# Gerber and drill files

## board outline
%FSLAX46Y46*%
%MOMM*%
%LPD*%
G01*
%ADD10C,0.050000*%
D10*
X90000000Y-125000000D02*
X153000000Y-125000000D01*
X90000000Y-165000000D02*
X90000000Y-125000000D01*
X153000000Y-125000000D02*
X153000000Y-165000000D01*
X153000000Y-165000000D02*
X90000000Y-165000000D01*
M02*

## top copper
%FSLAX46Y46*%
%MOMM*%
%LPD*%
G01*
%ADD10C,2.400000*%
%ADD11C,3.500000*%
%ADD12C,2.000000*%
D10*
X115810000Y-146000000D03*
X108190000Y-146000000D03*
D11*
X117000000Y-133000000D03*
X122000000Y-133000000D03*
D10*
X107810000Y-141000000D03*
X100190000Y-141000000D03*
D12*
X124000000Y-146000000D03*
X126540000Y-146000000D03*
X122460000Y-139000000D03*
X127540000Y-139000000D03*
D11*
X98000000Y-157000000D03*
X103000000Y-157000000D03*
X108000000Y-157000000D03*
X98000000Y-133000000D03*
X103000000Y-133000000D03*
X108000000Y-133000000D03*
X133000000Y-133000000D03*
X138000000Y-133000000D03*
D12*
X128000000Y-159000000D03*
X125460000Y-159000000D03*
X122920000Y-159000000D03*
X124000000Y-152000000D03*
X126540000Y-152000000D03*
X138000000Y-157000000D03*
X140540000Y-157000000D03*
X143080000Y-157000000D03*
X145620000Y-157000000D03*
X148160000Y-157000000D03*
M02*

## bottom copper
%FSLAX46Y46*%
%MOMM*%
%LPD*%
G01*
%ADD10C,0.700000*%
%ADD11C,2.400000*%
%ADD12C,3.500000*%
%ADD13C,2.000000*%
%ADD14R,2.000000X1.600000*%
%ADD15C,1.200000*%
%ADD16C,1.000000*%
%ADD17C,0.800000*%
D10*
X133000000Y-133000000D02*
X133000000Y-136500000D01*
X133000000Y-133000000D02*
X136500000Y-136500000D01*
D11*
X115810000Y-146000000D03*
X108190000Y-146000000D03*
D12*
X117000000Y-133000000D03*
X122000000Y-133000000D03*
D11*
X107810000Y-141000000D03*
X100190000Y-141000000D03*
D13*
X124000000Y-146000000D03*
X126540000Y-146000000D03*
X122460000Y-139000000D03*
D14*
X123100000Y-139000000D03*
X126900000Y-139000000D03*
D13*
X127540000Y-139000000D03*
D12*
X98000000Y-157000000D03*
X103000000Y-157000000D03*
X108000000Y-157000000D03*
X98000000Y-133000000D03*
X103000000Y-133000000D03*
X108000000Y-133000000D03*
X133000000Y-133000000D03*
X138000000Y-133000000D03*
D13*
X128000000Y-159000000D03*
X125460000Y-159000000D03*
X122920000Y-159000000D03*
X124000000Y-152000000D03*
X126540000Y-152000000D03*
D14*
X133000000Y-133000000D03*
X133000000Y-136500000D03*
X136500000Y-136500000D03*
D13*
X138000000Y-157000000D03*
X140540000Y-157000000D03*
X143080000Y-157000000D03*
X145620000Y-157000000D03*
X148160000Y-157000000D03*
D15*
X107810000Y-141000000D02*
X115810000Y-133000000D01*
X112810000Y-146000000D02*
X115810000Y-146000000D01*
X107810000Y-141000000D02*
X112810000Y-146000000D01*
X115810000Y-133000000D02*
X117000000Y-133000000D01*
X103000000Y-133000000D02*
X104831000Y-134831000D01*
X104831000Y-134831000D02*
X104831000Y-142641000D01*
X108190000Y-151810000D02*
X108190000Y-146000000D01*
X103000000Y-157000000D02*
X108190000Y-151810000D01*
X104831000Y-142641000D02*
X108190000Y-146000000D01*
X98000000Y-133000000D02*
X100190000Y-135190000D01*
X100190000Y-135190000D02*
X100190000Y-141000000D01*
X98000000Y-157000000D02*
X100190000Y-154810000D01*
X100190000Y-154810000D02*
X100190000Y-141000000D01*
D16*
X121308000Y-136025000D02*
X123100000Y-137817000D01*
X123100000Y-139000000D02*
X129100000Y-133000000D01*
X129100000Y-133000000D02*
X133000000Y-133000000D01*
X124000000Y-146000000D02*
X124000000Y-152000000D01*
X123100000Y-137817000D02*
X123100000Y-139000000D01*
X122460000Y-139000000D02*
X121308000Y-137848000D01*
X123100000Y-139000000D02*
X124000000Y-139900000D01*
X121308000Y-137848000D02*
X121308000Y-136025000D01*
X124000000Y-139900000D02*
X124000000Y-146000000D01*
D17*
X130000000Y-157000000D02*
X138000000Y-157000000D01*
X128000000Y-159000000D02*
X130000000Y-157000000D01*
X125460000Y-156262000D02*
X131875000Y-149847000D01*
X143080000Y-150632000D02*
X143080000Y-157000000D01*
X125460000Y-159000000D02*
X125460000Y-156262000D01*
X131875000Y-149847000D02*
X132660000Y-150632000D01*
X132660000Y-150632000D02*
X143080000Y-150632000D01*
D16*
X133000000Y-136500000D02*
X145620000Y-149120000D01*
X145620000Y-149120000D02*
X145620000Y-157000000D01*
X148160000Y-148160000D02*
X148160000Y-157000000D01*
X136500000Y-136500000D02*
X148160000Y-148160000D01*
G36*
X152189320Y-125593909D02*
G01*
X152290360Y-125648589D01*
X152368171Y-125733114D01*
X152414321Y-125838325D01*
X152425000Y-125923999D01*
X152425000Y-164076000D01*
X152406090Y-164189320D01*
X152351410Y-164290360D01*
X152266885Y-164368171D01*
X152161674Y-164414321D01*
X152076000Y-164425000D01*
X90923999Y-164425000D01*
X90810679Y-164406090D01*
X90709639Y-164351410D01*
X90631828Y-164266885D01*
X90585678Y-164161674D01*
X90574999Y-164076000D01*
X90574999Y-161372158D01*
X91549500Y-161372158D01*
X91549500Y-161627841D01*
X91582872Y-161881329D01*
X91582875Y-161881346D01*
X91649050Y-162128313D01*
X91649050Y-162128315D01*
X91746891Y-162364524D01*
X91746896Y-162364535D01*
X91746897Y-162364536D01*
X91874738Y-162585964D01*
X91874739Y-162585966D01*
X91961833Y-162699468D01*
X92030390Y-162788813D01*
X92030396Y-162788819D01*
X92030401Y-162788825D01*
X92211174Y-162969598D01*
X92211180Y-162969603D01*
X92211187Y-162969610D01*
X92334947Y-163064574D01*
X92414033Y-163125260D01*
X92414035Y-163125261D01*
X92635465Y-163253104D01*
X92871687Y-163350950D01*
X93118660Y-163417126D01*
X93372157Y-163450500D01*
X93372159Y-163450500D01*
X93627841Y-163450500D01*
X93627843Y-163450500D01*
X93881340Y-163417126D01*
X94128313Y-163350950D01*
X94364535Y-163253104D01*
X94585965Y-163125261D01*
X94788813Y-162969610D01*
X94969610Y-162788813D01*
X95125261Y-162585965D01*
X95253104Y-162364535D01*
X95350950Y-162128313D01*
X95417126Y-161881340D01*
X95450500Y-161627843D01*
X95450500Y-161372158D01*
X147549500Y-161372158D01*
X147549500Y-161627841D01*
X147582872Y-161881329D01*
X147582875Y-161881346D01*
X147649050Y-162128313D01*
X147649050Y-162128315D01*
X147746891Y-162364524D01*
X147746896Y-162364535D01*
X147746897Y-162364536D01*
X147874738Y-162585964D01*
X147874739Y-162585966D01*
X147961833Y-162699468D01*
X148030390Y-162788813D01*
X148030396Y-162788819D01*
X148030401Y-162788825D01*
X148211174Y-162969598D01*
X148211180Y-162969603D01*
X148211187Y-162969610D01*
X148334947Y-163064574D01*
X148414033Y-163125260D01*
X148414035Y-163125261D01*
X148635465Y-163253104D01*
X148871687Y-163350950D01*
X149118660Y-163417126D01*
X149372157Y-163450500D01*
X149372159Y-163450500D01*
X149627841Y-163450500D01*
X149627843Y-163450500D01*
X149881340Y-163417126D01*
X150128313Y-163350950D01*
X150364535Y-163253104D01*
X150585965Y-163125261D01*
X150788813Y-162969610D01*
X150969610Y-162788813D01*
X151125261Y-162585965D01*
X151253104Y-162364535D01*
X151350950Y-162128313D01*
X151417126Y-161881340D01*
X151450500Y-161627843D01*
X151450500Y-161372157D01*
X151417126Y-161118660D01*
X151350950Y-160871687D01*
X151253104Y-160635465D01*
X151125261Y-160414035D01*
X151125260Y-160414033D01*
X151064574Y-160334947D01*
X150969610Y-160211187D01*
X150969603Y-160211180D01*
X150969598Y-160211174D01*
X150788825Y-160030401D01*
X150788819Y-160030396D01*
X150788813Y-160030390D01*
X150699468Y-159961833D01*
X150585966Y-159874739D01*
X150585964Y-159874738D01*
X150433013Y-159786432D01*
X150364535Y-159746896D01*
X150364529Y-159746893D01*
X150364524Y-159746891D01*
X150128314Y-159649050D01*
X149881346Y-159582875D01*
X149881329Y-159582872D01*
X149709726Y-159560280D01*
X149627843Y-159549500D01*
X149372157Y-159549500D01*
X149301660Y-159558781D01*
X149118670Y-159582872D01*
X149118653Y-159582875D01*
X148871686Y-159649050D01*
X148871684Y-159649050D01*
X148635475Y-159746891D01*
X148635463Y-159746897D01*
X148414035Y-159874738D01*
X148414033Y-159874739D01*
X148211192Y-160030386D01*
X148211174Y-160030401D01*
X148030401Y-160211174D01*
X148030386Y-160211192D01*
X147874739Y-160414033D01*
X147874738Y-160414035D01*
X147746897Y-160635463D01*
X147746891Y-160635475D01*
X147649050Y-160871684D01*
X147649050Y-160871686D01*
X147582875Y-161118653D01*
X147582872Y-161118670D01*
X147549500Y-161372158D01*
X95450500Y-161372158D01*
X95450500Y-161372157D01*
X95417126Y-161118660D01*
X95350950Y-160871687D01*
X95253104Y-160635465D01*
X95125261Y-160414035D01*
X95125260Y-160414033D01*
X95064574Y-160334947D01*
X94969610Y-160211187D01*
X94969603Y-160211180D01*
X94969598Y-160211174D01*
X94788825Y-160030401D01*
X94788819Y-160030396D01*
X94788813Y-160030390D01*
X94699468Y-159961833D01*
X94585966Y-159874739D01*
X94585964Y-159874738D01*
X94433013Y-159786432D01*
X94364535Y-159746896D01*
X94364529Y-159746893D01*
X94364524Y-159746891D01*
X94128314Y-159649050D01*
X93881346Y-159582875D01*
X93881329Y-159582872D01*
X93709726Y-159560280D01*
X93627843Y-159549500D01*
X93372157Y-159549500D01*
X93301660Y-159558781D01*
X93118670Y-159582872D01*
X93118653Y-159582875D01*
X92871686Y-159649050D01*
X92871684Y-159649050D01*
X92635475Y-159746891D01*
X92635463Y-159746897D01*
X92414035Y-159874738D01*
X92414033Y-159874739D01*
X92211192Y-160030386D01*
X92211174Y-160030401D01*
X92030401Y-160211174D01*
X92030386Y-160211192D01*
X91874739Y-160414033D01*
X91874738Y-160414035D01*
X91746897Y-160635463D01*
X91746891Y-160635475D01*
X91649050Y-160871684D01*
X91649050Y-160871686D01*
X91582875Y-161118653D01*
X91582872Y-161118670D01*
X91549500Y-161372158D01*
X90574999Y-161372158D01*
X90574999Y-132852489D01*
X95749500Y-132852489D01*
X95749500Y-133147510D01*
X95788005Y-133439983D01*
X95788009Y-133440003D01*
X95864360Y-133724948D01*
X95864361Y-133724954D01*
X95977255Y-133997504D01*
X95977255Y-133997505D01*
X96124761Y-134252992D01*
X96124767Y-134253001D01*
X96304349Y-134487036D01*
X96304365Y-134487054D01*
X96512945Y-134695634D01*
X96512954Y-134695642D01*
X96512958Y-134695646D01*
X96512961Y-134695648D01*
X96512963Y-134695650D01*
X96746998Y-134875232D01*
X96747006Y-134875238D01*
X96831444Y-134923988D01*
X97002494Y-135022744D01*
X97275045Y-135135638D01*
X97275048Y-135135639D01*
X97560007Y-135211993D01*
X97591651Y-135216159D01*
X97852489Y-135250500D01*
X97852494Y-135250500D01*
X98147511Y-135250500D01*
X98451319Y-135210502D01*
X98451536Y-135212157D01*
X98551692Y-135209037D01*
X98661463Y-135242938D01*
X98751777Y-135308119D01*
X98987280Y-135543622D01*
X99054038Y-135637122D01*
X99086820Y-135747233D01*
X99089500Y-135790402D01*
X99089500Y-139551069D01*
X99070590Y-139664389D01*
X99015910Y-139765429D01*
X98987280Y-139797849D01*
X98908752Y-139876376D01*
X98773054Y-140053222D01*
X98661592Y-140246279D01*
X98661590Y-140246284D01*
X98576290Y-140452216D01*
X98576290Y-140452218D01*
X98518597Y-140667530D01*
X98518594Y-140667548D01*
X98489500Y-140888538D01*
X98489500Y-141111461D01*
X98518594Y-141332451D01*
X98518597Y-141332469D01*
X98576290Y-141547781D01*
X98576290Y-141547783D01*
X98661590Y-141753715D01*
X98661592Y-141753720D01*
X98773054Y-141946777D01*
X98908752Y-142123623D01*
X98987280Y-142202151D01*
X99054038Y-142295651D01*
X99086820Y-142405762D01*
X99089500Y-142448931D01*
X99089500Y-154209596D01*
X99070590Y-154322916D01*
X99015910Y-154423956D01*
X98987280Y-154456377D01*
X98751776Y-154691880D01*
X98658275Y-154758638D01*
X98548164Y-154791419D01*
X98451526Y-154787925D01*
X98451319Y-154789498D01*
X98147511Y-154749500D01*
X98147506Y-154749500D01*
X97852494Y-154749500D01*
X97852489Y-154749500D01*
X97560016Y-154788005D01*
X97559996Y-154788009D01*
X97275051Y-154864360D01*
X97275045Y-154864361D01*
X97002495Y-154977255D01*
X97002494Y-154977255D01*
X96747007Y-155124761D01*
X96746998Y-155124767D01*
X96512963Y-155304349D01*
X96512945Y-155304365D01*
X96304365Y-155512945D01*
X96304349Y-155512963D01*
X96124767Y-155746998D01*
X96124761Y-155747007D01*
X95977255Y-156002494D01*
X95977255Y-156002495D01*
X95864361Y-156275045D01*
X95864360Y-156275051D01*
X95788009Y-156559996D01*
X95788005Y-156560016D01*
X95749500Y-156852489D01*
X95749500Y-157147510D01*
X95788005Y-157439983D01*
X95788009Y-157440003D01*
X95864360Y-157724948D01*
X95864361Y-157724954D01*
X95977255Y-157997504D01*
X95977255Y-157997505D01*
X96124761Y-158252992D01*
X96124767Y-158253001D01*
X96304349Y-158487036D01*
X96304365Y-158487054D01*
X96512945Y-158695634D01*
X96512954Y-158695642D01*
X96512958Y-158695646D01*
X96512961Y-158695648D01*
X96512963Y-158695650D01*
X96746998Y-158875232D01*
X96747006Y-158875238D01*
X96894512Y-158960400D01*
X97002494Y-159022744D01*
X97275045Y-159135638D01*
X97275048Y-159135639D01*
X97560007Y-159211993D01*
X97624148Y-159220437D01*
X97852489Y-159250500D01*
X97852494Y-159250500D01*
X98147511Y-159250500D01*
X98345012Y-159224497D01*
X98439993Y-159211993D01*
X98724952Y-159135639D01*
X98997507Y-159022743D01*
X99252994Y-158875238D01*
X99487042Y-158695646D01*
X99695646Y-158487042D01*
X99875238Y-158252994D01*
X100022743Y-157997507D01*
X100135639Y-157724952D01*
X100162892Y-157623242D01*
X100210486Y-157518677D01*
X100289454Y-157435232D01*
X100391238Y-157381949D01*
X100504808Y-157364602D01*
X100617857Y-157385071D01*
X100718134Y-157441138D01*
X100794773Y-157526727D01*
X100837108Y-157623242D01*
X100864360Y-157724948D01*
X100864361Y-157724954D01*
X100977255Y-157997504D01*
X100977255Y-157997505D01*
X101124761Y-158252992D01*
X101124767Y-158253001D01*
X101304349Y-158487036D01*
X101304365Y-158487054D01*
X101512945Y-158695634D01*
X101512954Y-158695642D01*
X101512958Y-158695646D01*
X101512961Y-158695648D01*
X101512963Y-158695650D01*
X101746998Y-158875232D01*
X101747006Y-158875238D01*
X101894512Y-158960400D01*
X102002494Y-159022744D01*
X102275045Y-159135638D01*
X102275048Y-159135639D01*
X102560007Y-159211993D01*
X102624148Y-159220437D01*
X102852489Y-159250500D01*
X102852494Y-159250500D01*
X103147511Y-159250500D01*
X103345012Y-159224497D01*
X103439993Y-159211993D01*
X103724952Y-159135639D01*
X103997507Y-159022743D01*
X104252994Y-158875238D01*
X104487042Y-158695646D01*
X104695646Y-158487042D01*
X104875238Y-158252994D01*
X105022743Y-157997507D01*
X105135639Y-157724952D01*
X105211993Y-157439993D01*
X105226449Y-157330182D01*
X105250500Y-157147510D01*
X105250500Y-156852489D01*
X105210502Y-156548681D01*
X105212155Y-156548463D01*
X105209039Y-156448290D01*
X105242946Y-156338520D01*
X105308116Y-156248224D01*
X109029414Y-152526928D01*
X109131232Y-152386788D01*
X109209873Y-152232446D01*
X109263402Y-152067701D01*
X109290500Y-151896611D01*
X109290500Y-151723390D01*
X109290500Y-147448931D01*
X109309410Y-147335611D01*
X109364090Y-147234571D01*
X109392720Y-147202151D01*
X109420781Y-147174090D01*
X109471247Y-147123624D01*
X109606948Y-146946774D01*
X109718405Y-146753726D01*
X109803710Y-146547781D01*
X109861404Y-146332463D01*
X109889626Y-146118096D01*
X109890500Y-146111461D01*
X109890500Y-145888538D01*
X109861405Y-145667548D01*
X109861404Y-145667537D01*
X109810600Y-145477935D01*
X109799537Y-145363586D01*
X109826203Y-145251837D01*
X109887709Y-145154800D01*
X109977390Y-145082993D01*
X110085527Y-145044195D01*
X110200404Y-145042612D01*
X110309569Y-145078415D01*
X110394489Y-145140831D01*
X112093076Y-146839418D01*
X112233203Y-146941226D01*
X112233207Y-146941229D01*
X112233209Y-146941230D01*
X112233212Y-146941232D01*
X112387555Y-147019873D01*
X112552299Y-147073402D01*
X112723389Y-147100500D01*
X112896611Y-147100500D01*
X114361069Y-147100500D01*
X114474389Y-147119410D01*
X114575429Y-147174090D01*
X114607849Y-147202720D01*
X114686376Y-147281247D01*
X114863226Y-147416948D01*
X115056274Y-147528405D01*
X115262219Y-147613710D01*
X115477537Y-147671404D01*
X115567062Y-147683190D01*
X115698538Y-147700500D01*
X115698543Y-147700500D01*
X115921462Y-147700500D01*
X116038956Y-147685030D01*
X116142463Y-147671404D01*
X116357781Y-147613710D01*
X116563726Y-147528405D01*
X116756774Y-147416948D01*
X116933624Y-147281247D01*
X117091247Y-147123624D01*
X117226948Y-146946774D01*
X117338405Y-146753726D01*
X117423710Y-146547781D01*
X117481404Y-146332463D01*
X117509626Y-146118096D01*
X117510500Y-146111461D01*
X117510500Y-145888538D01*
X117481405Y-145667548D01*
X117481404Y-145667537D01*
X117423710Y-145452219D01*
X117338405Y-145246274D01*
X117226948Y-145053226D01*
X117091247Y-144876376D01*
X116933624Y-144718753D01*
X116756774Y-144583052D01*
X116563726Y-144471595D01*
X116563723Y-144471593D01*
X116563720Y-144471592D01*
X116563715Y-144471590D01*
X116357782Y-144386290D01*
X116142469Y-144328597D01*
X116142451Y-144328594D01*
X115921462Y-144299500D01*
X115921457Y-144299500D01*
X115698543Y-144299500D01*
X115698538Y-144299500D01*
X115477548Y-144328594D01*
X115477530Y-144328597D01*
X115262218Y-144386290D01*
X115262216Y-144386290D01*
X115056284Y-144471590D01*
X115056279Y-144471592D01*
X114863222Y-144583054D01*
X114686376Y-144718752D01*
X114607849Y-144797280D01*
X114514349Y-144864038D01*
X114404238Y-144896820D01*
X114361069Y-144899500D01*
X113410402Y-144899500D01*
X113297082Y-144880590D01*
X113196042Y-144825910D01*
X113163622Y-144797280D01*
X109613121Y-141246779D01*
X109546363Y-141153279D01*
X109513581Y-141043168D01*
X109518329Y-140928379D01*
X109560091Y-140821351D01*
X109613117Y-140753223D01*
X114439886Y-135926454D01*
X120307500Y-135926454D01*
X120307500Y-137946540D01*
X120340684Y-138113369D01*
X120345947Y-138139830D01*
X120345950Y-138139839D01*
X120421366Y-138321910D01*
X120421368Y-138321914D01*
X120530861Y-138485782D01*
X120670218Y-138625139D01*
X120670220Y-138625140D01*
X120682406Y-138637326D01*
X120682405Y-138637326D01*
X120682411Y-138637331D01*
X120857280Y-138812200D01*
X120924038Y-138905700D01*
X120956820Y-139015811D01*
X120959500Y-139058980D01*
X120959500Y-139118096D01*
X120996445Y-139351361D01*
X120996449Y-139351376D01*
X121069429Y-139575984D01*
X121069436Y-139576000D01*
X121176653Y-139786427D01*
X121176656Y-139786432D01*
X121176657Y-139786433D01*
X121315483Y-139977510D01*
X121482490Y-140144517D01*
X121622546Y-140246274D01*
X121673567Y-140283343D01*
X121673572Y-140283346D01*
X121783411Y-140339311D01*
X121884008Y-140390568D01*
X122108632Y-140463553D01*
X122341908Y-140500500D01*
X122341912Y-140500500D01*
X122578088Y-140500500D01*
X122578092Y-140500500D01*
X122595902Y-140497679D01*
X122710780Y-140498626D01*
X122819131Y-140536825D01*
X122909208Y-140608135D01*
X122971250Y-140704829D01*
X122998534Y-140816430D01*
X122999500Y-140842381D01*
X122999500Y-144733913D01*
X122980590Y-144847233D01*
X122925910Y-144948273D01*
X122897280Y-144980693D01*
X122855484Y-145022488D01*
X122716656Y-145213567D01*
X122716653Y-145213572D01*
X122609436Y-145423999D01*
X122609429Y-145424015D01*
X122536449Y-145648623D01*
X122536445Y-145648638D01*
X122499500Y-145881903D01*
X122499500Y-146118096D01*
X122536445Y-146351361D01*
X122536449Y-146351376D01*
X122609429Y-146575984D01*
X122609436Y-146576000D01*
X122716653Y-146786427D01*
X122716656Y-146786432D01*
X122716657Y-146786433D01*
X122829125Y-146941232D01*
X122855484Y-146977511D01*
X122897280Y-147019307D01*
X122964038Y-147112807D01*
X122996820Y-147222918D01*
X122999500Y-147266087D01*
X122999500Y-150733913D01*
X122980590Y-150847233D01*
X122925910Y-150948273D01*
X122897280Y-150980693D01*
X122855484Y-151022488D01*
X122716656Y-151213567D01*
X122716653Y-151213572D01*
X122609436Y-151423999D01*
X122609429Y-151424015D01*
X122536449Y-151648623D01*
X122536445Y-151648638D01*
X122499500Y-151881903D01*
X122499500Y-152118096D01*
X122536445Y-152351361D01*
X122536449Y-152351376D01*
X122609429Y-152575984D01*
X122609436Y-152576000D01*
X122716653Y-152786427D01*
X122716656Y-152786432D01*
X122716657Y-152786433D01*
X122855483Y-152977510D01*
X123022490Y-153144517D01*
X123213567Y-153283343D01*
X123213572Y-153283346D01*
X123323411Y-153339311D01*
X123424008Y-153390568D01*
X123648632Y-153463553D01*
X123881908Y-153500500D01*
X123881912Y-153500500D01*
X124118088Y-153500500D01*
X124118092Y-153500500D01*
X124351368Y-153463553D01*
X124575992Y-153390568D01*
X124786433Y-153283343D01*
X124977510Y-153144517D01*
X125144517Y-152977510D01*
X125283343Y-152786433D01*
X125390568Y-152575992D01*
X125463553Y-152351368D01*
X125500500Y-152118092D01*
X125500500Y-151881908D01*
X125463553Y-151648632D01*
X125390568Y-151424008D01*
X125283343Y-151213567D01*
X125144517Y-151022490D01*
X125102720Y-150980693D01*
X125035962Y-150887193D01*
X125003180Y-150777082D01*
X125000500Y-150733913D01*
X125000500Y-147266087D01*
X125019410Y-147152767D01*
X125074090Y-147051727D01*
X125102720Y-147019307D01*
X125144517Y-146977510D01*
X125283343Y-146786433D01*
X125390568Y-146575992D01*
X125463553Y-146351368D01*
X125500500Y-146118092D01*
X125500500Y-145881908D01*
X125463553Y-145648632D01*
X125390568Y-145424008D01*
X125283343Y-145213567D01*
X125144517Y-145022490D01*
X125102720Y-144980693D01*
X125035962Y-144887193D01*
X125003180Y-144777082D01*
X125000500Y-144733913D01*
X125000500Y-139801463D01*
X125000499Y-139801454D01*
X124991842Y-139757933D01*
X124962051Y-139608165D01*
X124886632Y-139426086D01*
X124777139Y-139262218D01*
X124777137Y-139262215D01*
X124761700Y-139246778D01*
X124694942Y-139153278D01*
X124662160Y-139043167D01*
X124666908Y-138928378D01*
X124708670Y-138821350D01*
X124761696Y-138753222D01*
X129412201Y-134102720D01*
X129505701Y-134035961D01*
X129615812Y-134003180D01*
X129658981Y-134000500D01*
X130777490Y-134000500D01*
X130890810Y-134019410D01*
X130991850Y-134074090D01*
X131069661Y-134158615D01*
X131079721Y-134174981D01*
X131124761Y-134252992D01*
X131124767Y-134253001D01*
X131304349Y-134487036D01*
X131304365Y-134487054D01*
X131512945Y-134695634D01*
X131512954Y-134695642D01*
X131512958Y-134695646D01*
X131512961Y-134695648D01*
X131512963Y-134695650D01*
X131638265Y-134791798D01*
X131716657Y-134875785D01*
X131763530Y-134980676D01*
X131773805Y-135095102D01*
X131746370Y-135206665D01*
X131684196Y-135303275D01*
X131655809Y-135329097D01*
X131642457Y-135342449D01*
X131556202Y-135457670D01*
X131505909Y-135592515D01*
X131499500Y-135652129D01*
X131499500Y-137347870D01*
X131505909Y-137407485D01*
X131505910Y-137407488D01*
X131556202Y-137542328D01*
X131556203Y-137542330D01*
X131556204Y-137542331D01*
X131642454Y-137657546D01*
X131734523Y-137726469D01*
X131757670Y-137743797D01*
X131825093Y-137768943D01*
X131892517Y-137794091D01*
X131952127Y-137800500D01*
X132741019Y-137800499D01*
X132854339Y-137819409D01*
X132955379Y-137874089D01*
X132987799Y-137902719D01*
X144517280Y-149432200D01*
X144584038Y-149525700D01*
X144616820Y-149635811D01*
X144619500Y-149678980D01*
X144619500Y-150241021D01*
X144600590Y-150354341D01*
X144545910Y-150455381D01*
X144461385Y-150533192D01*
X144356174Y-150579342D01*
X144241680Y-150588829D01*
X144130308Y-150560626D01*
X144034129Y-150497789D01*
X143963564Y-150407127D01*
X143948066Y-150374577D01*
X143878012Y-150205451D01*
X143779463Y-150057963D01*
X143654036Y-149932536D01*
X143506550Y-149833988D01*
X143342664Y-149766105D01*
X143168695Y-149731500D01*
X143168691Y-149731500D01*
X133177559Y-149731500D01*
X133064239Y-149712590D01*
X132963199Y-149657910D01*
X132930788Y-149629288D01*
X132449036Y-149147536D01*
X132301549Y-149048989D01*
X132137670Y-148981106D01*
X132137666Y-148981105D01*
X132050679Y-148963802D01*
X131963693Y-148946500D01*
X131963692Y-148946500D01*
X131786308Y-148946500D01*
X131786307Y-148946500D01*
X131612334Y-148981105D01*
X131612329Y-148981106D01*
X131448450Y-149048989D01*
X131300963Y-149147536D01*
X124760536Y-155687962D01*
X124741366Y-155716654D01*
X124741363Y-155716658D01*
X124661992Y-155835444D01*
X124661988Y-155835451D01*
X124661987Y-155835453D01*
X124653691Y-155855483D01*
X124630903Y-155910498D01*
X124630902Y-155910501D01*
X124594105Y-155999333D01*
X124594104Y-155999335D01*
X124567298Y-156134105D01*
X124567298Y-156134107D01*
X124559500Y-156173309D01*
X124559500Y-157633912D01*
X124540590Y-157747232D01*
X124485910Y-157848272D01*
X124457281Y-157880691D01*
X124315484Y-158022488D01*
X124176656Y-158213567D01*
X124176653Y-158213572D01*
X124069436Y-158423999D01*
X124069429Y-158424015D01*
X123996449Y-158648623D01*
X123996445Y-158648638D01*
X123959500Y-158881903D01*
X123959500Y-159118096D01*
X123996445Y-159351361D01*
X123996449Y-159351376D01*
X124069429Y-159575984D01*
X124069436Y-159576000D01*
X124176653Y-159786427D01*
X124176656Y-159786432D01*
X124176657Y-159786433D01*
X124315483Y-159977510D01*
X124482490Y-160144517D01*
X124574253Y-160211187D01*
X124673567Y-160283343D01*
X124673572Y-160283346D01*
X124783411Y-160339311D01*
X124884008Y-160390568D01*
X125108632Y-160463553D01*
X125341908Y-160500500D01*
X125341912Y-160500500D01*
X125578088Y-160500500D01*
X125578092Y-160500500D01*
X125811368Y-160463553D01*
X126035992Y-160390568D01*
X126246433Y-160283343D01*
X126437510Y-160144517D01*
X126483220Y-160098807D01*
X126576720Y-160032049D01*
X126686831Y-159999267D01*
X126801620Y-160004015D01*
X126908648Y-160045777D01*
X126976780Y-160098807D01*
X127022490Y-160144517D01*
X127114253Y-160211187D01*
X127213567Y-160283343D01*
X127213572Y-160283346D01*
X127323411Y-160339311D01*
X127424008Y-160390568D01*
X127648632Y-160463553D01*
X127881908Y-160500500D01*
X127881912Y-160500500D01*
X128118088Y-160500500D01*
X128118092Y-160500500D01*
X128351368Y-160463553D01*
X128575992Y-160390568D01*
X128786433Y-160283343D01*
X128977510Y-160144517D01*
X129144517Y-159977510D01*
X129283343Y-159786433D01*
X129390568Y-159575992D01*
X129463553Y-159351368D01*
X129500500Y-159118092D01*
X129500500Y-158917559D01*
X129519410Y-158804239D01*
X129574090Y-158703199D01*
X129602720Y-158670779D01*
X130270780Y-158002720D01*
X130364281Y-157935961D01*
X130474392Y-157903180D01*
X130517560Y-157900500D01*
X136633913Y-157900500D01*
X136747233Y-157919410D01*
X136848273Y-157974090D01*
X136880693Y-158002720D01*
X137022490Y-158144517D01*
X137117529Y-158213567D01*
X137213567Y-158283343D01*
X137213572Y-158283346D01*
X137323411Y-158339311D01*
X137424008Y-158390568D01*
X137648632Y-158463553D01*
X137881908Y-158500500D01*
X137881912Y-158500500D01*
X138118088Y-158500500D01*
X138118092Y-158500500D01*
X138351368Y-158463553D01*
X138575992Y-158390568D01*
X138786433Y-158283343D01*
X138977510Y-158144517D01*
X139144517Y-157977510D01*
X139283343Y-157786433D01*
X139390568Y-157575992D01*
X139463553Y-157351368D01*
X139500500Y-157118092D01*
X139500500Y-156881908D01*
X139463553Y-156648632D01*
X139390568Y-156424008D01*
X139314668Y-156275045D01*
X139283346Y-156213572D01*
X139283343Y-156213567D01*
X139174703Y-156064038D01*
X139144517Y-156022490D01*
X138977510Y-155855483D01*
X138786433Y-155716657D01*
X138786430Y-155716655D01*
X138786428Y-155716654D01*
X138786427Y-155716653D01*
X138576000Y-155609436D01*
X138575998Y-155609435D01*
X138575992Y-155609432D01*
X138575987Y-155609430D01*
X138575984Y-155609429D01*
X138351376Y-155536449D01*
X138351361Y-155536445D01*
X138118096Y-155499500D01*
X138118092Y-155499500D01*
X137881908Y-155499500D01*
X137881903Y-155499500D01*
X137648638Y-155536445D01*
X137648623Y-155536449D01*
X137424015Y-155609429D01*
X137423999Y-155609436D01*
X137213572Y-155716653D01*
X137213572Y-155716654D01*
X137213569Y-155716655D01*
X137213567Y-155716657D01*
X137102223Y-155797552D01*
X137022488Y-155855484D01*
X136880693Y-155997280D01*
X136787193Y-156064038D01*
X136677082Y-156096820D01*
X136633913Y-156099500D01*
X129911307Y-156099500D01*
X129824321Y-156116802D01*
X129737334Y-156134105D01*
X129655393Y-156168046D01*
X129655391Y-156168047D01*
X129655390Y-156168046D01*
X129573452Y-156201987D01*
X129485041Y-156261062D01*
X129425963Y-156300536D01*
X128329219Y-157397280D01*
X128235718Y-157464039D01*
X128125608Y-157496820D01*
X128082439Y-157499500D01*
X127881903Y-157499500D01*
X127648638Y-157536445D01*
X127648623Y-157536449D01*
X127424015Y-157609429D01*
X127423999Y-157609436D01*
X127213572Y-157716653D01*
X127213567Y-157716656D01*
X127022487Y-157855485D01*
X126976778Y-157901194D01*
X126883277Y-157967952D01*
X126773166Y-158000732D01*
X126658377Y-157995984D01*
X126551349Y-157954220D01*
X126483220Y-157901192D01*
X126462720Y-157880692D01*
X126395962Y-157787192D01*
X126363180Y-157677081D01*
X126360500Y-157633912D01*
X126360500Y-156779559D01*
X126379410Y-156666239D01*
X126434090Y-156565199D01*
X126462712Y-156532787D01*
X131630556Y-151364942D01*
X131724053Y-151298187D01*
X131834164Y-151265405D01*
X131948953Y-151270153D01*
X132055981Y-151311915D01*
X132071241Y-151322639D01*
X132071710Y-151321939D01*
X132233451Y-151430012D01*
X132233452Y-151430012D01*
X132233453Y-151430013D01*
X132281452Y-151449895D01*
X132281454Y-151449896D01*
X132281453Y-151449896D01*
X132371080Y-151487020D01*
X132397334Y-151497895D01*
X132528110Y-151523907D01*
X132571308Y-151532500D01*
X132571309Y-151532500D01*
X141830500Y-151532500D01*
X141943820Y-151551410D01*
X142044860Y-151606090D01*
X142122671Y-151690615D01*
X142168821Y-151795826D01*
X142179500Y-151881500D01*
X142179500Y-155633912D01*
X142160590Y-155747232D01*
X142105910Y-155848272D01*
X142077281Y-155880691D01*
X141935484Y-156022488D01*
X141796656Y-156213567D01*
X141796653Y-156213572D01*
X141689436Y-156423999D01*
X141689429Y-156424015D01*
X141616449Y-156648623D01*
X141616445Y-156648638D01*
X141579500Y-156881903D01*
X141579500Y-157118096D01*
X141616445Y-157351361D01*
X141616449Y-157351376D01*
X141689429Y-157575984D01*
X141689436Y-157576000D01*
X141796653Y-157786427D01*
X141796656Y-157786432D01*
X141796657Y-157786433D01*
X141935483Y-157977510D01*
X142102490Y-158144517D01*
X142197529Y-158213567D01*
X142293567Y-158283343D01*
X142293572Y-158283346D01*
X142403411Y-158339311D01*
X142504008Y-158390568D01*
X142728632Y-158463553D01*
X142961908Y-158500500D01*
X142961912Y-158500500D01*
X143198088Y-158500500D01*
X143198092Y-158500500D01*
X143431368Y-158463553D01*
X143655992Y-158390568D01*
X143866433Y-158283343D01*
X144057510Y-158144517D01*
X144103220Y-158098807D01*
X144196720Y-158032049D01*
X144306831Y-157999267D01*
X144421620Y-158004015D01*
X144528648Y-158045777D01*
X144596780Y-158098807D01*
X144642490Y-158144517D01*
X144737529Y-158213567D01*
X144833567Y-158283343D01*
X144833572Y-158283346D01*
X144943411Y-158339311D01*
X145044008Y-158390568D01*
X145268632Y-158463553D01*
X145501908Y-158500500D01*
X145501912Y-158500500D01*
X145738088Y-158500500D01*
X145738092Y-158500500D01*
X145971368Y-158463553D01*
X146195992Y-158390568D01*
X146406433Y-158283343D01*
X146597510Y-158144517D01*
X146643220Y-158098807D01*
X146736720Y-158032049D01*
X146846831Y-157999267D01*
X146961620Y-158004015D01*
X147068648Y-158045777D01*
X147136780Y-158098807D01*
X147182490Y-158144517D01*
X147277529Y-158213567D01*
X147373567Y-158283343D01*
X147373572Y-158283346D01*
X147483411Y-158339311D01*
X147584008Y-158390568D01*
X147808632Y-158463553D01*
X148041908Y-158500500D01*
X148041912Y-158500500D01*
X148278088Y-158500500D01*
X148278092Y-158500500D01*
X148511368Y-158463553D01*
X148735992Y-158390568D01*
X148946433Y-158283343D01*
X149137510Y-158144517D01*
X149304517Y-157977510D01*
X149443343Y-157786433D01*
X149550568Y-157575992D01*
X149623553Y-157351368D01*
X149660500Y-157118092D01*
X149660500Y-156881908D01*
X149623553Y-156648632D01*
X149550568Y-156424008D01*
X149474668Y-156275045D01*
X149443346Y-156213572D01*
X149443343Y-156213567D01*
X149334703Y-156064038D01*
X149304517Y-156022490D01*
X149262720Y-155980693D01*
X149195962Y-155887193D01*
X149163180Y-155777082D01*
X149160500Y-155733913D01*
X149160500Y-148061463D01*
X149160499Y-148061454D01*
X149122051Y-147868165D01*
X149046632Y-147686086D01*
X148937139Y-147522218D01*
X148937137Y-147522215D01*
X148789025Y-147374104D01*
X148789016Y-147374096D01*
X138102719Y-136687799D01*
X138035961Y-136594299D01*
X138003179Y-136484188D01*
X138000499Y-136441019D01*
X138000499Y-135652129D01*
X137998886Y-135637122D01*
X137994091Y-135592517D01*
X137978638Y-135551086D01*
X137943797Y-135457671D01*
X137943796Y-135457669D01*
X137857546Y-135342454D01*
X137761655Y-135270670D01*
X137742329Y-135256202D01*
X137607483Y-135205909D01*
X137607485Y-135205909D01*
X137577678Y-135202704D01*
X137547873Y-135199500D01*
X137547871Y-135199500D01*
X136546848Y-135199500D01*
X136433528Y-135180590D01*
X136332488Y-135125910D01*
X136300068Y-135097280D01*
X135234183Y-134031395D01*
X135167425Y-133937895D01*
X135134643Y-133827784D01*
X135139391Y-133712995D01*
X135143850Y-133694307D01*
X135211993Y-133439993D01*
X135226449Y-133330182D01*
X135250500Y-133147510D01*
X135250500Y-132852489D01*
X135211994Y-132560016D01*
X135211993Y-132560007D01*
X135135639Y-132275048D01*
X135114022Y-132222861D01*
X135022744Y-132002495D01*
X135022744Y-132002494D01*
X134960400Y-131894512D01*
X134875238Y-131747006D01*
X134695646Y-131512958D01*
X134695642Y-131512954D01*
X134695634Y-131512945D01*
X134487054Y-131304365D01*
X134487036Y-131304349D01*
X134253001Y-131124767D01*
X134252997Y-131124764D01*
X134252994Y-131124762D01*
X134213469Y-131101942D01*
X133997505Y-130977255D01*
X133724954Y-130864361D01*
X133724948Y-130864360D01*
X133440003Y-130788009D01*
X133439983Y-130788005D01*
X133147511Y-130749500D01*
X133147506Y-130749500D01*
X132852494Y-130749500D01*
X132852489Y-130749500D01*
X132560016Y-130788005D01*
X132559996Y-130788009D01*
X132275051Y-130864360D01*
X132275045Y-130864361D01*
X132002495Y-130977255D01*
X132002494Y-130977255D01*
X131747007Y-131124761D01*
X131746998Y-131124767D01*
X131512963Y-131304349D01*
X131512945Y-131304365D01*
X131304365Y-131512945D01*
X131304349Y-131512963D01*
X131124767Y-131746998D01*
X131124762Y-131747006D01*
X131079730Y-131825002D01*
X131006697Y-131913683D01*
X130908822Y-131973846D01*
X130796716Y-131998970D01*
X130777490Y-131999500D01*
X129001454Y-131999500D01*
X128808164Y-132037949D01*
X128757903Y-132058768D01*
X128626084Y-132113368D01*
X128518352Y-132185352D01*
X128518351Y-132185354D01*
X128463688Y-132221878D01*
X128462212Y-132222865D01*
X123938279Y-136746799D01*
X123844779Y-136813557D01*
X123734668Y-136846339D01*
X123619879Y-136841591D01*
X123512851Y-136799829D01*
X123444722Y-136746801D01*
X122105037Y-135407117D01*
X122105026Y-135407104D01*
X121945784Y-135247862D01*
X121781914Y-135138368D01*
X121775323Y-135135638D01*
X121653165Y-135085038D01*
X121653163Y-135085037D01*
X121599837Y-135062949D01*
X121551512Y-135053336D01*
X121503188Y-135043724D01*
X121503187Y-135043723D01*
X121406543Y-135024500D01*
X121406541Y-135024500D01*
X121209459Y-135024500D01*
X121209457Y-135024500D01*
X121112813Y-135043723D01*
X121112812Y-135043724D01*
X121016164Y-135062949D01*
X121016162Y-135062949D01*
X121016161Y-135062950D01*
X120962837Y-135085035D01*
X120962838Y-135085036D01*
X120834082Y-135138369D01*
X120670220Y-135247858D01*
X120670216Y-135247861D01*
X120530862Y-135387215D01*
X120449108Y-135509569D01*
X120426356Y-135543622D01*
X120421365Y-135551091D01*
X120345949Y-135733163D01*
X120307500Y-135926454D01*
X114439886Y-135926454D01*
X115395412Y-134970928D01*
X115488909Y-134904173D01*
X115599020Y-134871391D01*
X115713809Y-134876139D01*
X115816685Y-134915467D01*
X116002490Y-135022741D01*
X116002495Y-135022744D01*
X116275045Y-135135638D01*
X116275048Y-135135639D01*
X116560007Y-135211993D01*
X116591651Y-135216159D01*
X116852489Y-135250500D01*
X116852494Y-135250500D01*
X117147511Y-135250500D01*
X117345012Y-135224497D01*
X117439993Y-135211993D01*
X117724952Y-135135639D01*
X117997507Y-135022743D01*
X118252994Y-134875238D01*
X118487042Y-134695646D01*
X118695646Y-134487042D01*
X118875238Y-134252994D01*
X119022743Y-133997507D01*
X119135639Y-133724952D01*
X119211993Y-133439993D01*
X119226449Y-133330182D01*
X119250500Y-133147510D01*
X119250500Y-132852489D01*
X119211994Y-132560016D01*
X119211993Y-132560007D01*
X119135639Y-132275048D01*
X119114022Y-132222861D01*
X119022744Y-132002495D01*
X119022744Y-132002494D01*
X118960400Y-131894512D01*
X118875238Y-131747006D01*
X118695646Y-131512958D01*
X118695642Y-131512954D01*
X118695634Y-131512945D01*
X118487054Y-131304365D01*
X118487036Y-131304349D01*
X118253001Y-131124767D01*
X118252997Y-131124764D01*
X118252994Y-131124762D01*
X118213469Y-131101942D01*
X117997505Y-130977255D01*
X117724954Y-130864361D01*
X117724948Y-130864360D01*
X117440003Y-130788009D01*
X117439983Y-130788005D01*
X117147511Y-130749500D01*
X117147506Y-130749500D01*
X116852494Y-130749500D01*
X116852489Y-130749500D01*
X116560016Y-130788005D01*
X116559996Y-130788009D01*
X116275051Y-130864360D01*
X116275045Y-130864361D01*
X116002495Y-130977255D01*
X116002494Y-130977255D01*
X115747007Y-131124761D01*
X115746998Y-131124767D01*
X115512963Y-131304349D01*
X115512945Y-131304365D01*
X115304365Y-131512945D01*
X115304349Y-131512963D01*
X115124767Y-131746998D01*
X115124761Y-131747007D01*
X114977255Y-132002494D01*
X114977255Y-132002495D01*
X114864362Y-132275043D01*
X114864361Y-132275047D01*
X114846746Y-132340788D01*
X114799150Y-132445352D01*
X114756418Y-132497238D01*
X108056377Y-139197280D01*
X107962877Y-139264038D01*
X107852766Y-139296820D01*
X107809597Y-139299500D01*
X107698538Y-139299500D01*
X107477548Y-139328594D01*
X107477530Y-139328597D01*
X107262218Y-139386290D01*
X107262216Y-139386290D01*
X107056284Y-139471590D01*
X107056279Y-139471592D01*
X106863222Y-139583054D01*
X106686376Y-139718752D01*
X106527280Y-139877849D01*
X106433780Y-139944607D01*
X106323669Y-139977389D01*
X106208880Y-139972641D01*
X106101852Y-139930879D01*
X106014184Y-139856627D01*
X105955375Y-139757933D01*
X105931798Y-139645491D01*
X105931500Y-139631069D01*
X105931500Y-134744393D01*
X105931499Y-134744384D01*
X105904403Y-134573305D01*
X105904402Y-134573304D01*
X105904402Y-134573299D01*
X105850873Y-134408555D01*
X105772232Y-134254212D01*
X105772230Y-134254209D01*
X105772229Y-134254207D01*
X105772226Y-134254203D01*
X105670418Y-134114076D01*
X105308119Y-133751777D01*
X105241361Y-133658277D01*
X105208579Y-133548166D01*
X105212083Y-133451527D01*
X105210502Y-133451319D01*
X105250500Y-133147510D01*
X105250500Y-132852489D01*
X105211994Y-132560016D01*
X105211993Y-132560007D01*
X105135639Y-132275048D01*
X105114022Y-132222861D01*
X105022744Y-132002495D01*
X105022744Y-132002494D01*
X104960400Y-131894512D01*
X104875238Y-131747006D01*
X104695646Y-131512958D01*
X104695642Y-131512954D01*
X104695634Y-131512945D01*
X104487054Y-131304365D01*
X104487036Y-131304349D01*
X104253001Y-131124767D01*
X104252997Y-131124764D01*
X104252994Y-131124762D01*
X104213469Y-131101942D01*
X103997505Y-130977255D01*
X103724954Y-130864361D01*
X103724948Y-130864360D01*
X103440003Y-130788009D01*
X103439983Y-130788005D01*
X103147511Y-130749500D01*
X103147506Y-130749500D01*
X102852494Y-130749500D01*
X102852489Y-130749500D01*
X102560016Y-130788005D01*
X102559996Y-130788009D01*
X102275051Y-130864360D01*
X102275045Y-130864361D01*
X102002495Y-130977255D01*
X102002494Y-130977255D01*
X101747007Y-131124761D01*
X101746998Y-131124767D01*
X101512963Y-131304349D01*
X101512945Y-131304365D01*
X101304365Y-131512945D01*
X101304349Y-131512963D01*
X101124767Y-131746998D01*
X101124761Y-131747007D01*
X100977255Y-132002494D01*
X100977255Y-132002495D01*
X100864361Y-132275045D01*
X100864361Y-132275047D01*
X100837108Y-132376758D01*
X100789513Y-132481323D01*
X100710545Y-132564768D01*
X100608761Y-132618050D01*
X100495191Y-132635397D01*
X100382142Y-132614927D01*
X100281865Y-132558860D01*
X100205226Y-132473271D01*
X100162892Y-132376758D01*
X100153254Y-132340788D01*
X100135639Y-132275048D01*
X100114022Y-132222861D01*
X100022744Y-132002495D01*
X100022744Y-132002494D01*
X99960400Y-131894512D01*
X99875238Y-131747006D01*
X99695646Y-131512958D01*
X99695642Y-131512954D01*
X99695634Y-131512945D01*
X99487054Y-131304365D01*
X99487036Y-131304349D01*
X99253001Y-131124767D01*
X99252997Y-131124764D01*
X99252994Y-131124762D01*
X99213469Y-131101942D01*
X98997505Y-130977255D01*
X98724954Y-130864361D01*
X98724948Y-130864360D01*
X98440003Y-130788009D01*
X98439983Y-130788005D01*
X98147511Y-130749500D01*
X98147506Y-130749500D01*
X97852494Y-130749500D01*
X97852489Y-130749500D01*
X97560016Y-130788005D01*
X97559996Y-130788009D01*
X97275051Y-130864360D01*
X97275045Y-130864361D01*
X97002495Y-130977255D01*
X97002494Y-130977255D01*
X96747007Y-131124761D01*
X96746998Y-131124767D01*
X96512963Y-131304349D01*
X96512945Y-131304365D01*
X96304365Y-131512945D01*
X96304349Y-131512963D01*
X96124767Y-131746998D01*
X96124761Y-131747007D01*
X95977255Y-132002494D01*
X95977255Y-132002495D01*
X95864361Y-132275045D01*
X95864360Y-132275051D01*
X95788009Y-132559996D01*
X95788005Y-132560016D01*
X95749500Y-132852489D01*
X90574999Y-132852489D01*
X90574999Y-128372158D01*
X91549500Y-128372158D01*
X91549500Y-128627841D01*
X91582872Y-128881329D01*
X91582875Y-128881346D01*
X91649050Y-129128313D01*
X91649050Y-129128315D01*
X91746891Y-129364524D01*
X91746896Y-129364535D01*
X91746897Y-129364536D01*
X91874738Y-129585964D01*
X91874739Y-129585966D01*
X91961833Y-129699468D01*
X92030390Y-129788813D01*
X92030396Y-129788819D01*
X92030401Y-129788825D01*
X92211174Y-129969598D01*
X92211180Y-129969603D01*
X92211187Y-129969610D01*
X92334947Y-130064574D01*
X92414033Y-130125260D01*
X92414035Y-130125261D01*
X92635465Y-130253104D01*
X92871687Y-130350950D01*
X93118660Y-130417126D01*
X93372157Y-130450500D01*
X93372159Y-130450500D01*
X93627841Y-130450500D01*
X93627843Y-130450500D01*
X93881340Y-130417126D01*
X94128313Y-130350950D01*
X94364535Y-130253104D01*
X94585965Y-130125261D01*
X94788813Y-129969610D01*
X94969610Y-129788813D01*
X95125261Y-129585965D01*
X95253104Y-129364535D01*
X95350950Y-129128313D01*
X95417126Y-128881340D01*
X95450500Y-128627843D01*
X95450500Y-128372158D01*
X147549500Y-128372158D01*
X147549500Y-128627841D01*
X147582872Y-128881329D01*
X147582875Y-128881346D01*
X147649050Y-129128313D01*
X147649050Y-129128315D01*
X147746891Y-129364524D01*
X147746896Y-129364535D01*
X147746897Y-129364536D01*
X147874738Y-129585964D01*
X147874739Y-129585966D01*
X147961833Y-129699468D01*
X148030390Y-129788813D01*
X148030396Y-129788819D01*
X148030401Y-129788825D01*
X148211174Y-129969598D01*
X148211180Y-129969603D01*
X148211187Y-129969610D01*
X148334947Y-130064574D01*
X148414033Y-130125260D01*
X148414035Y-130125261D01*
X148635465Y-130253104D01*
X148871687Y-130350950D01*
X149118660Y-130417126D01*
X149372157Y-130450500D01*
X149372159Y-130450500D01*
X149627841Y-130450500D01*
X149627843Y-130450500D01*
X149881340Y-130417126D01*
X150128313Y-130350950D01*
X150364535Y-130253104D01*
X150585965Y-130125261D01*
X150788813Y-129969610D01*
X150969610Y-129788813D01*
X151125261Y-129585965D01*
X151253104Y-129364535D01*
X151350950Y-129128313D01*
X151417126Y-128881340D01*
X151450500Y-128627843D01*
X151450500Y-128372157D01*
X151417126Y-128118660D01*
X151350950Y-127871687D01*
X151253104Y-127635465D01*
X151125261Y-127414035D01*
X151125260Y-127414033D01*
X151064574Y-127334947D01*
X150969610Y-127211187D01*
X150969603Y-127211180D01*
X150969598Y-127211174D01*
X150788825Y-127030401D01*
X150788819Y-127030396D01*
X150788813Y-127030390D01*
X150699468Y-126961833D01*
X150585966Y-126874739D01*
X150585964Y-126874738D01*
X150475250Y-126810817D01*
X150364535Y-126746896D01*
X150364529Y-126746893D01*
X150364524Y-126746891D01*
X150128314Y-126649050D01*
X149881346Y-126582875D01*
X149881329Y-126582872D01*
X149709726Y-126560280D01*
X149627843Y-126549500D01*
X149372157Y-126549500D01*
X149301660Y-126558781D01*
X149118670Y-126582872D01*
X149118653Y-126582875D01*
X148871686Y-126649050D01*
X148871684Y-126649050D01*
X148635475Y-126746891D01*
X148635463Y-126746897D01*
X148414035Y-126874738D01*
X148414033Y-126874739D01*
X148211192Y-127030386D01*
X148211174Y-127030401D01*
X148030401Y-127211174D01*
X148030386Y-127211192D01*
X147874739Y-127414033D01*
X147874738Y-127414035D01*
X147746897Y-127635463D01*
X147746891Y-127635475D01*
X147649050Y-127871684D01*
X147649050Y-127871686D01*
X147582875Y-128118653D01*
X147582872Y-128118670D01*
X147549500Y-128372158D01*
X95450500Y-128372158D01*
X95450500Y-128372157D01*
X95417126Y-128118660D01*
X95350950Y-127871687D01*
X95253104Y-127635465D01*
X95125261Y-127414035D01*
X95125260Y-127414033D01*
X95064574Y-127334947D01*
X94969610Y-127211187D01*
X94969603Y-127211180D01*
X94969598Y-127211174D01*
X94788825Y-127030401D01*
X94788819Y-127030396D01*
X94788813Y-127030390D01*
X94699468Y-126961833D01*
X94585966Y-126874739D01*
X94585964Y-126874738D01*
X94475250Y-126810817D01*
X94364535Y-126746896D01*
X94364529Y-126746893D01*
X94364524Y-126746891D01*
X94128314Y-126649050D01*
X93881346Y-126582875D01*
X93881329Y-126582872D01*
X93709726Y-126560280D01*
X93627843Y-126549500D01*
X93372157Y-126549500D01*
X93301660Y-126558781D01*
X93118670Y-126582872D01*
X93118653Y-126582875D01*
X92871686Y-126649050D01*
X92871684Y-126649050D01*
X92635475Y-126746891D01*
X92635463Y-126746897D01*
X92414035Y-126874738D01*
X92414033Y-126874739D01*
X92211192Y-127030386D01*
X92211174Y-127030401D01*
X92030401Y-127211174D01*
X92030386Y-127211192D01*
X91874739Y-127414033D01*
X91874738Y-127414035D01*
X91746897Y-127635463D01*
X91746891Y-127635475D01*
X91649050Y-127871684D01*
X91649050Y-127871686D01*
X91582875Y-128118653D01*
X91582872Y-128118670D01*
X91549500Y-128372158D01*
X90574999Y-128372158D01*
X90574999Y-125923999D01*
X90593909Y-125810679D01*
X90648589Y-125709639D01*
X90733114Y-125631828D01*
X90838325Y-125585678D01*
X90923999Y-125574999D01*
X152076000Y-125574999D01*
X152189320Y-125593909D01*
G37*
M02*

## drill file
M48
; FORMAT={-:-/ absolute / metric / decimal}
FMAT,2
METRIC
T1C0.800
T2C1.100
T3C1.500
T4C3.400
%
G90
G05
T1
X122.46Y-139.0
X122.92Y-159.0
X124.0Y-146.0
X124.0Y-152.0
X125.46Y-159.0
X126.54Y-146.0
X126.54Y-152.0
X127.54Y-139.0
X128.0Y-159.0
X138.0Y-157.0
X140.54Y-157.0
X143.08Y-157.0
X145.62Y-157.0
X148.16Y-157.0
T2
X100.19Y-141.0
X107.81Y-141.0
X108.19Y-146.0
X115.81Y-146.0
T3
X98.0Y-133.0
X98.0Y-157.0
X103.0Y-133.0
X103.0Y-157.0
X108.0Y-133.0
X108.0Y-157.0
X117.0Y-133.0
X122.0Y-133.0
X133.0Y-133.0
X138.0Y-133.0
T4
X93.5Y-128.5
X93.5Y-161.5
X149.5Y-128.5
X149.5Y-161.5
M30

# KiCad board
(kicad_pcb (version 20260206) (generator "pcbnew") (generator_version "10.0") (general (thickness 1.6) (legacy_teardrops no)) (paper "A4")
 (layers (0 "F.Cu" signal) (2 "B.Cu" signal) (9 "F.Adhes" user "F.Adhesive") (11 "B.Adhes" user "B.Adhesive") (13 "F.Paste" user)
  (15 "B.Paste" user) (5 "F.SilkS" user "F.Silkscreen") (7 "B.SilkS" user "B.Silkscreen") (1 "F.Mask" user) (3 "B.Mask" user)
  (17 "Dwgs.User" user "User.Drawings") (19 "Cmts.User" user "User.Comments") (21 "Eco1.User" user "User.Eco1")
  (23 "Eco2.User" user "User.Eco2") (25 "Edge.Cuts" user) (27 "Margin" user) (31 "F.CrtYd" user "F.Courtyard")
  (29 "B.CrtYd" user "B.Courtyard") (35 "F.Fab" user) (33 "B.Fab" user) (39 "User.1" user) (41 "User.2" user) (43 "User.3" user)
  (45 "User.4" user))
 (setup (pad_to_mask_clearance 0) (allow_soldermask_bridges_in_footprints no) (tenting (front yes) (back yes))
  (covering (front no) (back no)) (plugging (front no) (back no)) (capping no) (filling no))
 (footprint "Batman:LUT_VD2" (layer "F.Cu") (at 112 146 180)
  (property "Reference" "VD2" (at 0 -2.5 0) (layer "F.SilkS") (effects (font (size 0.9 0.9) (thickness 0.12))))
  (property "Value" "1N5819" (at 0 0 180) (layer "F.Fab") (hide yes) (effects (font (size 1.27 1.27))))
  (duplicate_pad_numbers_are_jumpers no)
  (pad "1" thru_hole circle (at -3.81 0 180) (size 2.4 2.4) (drill 1.1) (layers "*.Cu") (remove_unused_layers no) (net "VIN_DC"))
  (pad "2" thru_hole circle (at 3.81 0 180) (size 2.4 2.4) (drill 1.1) (layers "*.Cu") (remove_unused_layers no) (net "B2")))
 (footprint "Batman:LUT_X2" (layer "F.Cu") (at 117 133)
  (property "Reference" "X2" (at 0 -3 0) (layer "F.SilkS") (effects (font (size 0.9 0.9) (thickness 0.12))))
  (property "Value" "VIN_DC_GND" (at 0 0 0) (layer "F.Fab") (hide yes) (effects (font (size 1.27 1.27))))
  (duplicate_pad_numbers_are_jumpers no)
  (pad "1" thru_hole circle (at 0 0) (size 3.5 3.5) (drill 1.5) (layers "*.Cu") (remove_unused_layers no) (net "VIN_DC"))
  (pad "2" thru_hole circle (at 5 0) (size 3.5 3.5) (drill 1.5) (layers "*.Cu") (remove_unused_layers no) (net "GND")))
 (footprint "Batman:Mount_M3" (layer "F.Cu") (at 149.5 128.5)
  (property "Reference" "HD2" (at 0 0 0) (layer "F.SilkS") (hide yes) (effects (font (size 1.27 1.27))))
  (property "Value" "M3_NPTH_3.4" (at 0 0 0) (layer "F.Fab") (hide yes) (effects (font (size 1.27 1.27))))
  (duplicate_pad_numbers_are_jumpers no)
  (pad "" np_thru_hole circle (at 0 0) (size 3.4 3.4) (drill 3.4) (layers "*.Cu")))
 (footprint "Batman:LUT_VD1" (layer "F.Cu") (at 104 141 180)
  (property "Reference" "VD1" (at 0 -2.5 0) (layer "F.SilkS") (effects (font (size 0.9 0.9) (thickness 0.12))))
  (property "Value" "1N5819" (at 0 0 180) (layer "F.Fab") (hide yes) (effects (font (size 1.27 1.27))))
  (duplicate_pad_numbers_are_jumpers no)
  (pad "1" thru_hole circle (at -3.81 0 180) (size 2.4 2.4) (drill 1.1) (layers "*.Cu") (remove_unused_layers no) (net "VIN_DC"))
  (pad "2" thru_hole circle (at 3.81 0 180) (size 2.4 2.4) (drill 1.1) (layers "*.Cu") (remove_unused_layers no) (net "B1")))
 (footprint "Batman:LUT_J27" (layer "F.Cu") (at 124 146)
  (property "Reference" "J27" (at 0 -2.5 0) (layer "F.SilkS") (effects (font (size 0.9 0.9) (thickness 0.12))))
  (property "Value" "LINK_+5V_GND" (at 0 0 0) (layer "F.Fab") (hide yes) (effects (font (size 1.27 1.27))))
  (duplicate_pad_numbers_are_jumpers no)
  (pad "1" thru_hole circle (at 0 0) (size 2 2) (drill 0.8) (layers "*.Cu") (remove_unused_layers no) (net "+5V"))
  (pad "2" thru_hole circle (at 2.54 0) (size 2 2) (drill 0.8) (layers "*.Cu") (remove_unused_layers no) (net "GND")))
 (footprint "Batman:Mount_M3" (layer "F.Cu") (at 93.5 128.5)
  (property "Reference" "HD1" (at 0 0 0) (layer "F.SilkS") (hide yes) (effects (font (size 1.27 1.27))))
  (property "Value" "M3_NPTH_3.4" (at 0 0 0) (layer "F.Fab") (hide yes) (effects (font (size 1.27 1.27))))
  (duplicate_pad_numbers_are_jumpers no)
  (pad "" np_thru_hole circle (at 0 0) (size 3.4 3.4) (drill 3.4) (layers "*.Cu")))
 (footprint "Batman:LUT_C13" (layer "F.Cu") (at 125 139)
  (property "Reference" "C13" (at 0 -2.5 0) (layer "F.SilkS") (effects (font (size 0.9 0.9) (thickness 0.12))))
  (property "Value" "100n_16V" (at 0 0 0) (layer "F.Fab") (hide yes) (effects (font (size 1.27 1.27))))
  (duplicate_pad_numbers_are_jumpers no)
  (pad "1" thru_hole circle (at -2.54 0) (size 2 2) (drill 0.8) (layers "*.Cu") (remove_unused_layers no) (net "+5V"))
  (pad "1" smd rect (at -1.9 0) (size 2 1.6) (layers "B.Cu") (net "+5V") (thermal_bridge_angle 45))
  (pad "2" smd rect (at 1.9 0) (size 2 1.6) (layers "B.Cu") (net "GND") (thermal_bridge_angle 45))
  (pad "2" thru_hole circle (at 2.54 0) (size 2 2) (drill 0.8) (layers "*.Cu") (remove_unused_layers no) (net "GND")))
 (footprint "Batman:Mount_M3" (layer "F.Cu") (at 93.5 161.5)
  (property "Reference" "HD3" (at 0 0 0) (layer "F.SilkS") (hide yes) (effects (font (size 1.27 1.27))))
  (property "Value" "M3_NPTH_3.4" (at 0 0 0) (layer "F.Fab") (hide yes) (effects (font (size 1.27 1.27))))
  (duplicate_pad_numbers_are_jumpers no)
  (pad "" np_thru_hole circle (at 0 0) (size 3.4 3.4) (drill 3.4) (layers "*.Cu")))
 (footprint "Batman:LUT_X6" (layer "F.Cu") (at 98 157)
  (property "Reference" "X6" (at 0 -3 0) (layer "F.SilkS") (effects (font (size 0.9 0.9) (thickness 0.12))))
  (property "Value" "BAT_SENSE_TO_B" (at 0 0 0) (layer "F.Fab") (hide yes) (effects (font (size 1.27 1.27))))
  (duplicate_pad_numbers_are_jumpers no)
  (pad "1" thru_hole circle (at 0 0) (size 3.5 3.5) (drill 1.5) (layers "*.Cu") (remove_unused_layers no) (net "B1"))
  (pad "2" thru_hole circle (at 5 0) (size 3.5 3.5) (drill 1.5) (layers "*.Cu") (remove_unused_layers no) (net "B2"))
  (pad "3" thru_hole circle (at 10 0) (size 3.5 3.5) (drill 1.5) (layers "*.Cu") (remove_unused_layers no) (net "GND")))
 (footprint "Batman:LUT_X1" (layer "F.Cu") (at 98 133)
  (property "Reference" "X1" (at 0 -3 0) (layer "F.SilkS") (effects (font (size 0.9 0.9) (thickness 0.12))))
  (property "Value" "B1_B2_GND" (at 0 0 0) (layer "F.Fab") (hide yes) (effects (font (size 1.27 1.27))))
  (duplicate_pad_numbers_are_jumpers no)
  (pad "1" thru_hole circle (at 0 0) (size 3.5 3.5) (drill 1.5) (layers "*.Cu") (remove_unused_layers no) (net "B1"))
  (pad "2" thru_hole circle (at 5 0) (size 3.5 3.5) (drill 1.5) (layers "*.Cu") (remove_unused_layers no) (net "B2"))
  (pad "3" thru_hole circle (at 10 0) (size 3.5 3.5) (drill 1.5) (layers "*.Cu") (remove_unused_layers no) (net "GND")))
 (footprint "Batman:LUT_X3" (layer "F.Cu") (at 133 133)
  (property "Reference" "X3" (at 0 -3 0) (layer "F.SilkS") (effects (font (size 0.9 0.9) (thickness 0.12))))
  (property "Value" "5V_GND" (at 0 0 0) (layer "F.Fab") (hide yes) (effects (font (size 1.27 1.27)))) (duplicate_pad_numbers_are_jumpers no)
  (pad "1" thru_hole circle (at 0 0) (size 3.5 3.5) (drill 1.5) (layers "*.Cu") (remove_unused_layers no) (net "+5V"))
  (pad "2" thru_hole circle (at 5 0) (size 3.5 3.5) (drill 1.5) (layers "*.Cu") (remove_unused_layers no) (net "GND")))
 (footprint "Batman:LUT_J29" (layer "F.Cu") (at 128 159 180)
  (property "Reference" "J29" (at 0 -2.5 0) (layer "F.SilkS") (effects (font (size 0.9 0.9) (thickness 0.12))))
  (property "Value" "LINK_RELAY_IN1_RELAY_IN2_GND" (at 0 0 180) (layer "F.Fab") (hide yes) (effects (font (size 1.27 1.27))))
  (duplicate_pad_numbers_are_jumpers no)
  (pad "1" thru_hole circle (at 0 0 180) (size 2 2) (drill 0.8) (layers "*.Cu") (remove_unused_layers no) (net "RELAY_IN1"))
  (pad "2" thru_hole circle (at 2.54 0 180) (size 2 2) (drill 0.8) (layers "*.Cu") (remove_unused_layers no) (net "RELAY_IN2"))
  (pad "3" thru_hole circle (at 5.08 0 180) (size 2 2) (drill 0.8) (layers "*.Cu") (remove_unused_layers no) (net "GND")))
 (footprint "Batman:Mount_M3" (layer "F.Cu") (at 149.5 161.5)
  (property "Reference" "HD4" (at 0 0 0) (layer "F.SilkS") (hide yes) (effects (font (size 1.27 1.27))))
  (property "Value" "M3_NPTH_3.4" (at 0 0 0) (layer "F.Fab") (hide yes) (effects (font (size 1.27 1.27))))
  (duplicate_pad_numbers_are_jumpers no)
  (pad "" np_thru_hole circle (at 0 0) (size 3.4 3.4) (drill 3.4) (layers "*.Cu")))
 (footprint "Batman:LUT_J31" (layer "F.Cu") (at 124 152)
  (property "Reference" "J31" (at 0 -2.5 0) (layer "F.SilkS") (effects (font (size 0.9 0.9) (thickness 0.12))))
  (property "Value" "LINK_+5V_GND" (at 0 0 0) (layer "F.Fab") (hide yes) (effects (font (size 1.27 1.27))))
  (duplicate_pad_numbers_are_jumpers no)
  (pad "1" thru_hole circle (at 0 0) (size 2 2) (drill 0.8) (layers "*.Cu") (remove_unused_layers no) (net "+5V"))
  (pad "2" thru_hole circle (at 2.54 0) (size 2 2) (drill 0.8) (layers "*.Cu") (remove_unused_layers no) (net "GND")))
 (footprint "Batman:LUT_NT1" (layer "F.Cu") (at 133 133)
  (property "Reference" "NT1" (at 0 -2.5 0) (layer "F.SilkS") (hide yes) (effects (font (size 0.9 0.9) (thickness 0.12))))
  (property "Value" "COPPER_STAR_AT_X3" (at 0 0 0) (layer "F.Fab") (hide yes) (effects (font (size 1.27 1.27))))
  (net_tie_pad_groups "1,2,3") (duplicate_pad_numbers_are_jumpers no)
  (fp_line (start 0 0) (end 0 3.5) (stroke (width 0.7) (type default)) (layer "B.Cu"))
  (fp_line (start 0 0) (end 3.5 3.5) (stroke (width 0.7) (type default)) (layer "B.Cu"))
  (pad "1" smd rect (at 0 0) (size 2 1.6) (layers "B.Cu") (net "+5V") (thermal_bridge_angle 45))
  (pad "2" smd rect (at 0 3.5) (size 2 1.6) (layers "B.Cu") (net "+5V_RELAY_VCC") (thermal_bridge_angle 45))
  (pad "3" smd rect (at 3.5 3.5) (size 2 1.6) (layers "B.Cu") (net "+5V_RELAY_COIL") (thermal_bridge_angle 45)))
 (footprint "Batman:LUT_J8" (layer "F.Cu") (at 138 157 90)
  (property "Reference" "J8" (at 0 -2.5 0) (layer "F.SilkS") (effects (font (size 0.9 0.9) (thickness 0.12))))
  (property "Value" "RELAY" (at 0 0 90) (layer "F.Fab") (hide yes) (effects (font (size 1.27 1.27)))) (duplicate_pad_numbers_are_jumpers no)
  (pad "1" thru_hole circle (at 0 0 90) (size 2 2) (drill 0.8) (layers "*.Cu") (remove_unused_layers no) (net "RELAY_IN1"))
  (pad "2" thru_hole circle (at 0 2.54 90) (size 2 2) (drill 0.8) (layers "*.Cu") (remove_unused_layers no) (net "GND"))
  (pad "3" thru_hole circle (at 0 5.08 90) (size 2 2) (drill 0.8) (layers "*.Cu") (remove_unused_layers no) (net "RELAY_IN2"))
  (pad "4" thru_hole circle (at 0 7.62 90) (size 2 2) (drill 0.8) (layers "*.Cu") (remove_unused_layers no) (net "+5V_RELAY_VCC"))
  (pad "5" thru_hole circle (at 0 10.16 90) (size 2 2) (drill 0.8) (layers "*.Cu") (remove_unused_layers no) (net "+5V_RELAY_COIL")))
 (gr_line (start 90 125) (end 153 125) (stroke (width 0.05) (type default)) (layer "Edge.Cuts"))
 (gr_line (start 90 165) (end 90 125) (stroke (width 0.05) (type default)) (layer "Edge.Cuts"))
 (gr_line (start 153 125) (end 153 165) (stroke (width 0.05) (type default)) (layer "Edge.Cuts"))
 (gr_line (start 153 165) (end 90 165) (stroke (width 0.05) (type default)) (layer "Edge.Cuts"))
 (segment (start 107.81 141) (end 115.81 133) (width 1.2) (layer "B.Cu") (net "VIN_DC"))
 (segment (start 112.81 146) (end 115.81 146) (width 1.2) (layer "B.Cu") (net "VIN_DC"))
 (segment (start 107.81 141) (end 112.81 146) (width 1.2) (layer "B.Cu") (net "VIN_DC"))
 (segment (start 115.81 133) (end 117 133) (width 1.2) (layer "B.Cu") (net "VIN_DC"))
 (segment (start 103 133) (end 104.831 134.831) (width 1.2) (layer "B.Cu") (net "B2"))
 (segment (start 104.831 134.831) (end 104.831 142.641) (width 1.2) (layer "B.Cu") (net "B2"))
 (segment (start 108.19 151.81) (end 108.19 146) (width 1.2) (layer "B.Cu") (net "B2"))
 (segment (start 103 157) (end 108.19 151.81) (width 1.2) (layer "B.Cu") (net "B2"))
 (segment (start 104.831 142.641) (end 108.19 146) (width 1.2) (layer "B.Cu") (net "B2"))
 (segment (start 98 133) (end 100.19 135.19) (width 1.2) (layer "B.Cu") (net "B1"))
 (segment (start 100.19 135.19) (end 100.19 141) (width 1.2) (layer "B.Cu") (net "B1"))
 (segment (start 98 157) (end 100.19 154.81) (width 1.2) (layer "B.Cu") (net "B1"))
 (segment (start 100.19 154.81) (end 100.19 141) (width 1.2) (layer "B.Cu") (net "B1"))
 (segment (start 121.308 136.025) (end 123.1 137.817) (width 1) (layer "B.Cu") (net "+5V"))
 (segment (start 123.1 139) (end 129.1 133) (width 1) (layer "B.Cu") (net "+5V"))
 (segment (start 129.1 133) (end 133 133) (width 1) (layer "B.Cu") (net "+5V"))
 (segment (start 124 146) (end 124 152) (width 1) (layer "B.Cu") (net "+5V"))
 (segment (start 123.1 137.817) (end 123.1 139) (width 1) (layer "B.Cu") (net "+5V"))
 (segment (start 122.46 139) (end 121.308 137.848) (width 1) (layer "B.Cu") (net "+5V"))
 (segment (start 123.1 139) (end 124 139.9) (width 1) (layer "B.Cu") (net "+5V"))
 (segment (start 121.308 137.848) (end 121.308 136.025) (width 1) (layer "B.Cu") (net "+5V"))
 (segment (start 124 139.9) (end 124 146) (width 1) (layer "B.Cu") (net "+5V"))
 (segment (start 130 157) (end 138 157) (width 0.8) (layer "B.Cu") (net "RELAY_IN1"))
 (segment (start 128 159) (end 130 157) (width 0.8) (layer "B.Cu") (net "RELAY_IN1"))
 (segment (start 125.46 156.262) (end 131.875 149.847) (width 0.8) (layer "B.Cu") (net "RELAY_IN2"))
 (segment (start 143.08 150.632) (end 143.08 157) (width 0.8) (layer "B.Cu") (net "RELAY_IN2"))
 (segment (start 125.46 159) (end 125.46 156.262) (width 0.8) (layer "B.Cu") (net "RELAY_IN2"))
 (segment (start 131.875 149.847) (end 132.66 150.632) (width 0.8) (layer "B.Cu") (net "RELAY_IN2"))
 (segment (start 132.66 150.632) (end 143.08 150.632) (width 0.8) (layer "B.Cu") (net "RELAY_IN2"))
 (segment (start 133 136.5) (end 145.62 149.12) (width 1) (layer "B.Cu") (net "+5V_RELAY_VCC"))
 (segment (start 145.62 149.12) (end 145.62 157) (width 1) (layer "B.Cu") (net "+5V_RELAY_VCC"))
 (segment (start 148.16 148.16) (end 148.16 157) (width 1) (layer "B.Cu") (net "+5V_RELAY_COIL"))
 (segment (start 136.5 136.5) (end 148.16 148.16) (width 1) (layer "B.Cu") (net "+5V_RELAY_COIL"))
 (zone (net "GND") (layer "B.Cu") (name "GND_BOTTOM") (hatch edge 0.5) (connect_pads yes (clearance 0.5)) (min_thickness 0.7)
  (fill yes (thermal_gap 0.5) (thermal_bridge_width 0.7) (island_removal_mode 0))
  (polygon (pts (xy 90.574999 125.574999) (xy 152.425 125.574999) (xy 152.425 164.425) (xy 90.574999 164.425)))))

